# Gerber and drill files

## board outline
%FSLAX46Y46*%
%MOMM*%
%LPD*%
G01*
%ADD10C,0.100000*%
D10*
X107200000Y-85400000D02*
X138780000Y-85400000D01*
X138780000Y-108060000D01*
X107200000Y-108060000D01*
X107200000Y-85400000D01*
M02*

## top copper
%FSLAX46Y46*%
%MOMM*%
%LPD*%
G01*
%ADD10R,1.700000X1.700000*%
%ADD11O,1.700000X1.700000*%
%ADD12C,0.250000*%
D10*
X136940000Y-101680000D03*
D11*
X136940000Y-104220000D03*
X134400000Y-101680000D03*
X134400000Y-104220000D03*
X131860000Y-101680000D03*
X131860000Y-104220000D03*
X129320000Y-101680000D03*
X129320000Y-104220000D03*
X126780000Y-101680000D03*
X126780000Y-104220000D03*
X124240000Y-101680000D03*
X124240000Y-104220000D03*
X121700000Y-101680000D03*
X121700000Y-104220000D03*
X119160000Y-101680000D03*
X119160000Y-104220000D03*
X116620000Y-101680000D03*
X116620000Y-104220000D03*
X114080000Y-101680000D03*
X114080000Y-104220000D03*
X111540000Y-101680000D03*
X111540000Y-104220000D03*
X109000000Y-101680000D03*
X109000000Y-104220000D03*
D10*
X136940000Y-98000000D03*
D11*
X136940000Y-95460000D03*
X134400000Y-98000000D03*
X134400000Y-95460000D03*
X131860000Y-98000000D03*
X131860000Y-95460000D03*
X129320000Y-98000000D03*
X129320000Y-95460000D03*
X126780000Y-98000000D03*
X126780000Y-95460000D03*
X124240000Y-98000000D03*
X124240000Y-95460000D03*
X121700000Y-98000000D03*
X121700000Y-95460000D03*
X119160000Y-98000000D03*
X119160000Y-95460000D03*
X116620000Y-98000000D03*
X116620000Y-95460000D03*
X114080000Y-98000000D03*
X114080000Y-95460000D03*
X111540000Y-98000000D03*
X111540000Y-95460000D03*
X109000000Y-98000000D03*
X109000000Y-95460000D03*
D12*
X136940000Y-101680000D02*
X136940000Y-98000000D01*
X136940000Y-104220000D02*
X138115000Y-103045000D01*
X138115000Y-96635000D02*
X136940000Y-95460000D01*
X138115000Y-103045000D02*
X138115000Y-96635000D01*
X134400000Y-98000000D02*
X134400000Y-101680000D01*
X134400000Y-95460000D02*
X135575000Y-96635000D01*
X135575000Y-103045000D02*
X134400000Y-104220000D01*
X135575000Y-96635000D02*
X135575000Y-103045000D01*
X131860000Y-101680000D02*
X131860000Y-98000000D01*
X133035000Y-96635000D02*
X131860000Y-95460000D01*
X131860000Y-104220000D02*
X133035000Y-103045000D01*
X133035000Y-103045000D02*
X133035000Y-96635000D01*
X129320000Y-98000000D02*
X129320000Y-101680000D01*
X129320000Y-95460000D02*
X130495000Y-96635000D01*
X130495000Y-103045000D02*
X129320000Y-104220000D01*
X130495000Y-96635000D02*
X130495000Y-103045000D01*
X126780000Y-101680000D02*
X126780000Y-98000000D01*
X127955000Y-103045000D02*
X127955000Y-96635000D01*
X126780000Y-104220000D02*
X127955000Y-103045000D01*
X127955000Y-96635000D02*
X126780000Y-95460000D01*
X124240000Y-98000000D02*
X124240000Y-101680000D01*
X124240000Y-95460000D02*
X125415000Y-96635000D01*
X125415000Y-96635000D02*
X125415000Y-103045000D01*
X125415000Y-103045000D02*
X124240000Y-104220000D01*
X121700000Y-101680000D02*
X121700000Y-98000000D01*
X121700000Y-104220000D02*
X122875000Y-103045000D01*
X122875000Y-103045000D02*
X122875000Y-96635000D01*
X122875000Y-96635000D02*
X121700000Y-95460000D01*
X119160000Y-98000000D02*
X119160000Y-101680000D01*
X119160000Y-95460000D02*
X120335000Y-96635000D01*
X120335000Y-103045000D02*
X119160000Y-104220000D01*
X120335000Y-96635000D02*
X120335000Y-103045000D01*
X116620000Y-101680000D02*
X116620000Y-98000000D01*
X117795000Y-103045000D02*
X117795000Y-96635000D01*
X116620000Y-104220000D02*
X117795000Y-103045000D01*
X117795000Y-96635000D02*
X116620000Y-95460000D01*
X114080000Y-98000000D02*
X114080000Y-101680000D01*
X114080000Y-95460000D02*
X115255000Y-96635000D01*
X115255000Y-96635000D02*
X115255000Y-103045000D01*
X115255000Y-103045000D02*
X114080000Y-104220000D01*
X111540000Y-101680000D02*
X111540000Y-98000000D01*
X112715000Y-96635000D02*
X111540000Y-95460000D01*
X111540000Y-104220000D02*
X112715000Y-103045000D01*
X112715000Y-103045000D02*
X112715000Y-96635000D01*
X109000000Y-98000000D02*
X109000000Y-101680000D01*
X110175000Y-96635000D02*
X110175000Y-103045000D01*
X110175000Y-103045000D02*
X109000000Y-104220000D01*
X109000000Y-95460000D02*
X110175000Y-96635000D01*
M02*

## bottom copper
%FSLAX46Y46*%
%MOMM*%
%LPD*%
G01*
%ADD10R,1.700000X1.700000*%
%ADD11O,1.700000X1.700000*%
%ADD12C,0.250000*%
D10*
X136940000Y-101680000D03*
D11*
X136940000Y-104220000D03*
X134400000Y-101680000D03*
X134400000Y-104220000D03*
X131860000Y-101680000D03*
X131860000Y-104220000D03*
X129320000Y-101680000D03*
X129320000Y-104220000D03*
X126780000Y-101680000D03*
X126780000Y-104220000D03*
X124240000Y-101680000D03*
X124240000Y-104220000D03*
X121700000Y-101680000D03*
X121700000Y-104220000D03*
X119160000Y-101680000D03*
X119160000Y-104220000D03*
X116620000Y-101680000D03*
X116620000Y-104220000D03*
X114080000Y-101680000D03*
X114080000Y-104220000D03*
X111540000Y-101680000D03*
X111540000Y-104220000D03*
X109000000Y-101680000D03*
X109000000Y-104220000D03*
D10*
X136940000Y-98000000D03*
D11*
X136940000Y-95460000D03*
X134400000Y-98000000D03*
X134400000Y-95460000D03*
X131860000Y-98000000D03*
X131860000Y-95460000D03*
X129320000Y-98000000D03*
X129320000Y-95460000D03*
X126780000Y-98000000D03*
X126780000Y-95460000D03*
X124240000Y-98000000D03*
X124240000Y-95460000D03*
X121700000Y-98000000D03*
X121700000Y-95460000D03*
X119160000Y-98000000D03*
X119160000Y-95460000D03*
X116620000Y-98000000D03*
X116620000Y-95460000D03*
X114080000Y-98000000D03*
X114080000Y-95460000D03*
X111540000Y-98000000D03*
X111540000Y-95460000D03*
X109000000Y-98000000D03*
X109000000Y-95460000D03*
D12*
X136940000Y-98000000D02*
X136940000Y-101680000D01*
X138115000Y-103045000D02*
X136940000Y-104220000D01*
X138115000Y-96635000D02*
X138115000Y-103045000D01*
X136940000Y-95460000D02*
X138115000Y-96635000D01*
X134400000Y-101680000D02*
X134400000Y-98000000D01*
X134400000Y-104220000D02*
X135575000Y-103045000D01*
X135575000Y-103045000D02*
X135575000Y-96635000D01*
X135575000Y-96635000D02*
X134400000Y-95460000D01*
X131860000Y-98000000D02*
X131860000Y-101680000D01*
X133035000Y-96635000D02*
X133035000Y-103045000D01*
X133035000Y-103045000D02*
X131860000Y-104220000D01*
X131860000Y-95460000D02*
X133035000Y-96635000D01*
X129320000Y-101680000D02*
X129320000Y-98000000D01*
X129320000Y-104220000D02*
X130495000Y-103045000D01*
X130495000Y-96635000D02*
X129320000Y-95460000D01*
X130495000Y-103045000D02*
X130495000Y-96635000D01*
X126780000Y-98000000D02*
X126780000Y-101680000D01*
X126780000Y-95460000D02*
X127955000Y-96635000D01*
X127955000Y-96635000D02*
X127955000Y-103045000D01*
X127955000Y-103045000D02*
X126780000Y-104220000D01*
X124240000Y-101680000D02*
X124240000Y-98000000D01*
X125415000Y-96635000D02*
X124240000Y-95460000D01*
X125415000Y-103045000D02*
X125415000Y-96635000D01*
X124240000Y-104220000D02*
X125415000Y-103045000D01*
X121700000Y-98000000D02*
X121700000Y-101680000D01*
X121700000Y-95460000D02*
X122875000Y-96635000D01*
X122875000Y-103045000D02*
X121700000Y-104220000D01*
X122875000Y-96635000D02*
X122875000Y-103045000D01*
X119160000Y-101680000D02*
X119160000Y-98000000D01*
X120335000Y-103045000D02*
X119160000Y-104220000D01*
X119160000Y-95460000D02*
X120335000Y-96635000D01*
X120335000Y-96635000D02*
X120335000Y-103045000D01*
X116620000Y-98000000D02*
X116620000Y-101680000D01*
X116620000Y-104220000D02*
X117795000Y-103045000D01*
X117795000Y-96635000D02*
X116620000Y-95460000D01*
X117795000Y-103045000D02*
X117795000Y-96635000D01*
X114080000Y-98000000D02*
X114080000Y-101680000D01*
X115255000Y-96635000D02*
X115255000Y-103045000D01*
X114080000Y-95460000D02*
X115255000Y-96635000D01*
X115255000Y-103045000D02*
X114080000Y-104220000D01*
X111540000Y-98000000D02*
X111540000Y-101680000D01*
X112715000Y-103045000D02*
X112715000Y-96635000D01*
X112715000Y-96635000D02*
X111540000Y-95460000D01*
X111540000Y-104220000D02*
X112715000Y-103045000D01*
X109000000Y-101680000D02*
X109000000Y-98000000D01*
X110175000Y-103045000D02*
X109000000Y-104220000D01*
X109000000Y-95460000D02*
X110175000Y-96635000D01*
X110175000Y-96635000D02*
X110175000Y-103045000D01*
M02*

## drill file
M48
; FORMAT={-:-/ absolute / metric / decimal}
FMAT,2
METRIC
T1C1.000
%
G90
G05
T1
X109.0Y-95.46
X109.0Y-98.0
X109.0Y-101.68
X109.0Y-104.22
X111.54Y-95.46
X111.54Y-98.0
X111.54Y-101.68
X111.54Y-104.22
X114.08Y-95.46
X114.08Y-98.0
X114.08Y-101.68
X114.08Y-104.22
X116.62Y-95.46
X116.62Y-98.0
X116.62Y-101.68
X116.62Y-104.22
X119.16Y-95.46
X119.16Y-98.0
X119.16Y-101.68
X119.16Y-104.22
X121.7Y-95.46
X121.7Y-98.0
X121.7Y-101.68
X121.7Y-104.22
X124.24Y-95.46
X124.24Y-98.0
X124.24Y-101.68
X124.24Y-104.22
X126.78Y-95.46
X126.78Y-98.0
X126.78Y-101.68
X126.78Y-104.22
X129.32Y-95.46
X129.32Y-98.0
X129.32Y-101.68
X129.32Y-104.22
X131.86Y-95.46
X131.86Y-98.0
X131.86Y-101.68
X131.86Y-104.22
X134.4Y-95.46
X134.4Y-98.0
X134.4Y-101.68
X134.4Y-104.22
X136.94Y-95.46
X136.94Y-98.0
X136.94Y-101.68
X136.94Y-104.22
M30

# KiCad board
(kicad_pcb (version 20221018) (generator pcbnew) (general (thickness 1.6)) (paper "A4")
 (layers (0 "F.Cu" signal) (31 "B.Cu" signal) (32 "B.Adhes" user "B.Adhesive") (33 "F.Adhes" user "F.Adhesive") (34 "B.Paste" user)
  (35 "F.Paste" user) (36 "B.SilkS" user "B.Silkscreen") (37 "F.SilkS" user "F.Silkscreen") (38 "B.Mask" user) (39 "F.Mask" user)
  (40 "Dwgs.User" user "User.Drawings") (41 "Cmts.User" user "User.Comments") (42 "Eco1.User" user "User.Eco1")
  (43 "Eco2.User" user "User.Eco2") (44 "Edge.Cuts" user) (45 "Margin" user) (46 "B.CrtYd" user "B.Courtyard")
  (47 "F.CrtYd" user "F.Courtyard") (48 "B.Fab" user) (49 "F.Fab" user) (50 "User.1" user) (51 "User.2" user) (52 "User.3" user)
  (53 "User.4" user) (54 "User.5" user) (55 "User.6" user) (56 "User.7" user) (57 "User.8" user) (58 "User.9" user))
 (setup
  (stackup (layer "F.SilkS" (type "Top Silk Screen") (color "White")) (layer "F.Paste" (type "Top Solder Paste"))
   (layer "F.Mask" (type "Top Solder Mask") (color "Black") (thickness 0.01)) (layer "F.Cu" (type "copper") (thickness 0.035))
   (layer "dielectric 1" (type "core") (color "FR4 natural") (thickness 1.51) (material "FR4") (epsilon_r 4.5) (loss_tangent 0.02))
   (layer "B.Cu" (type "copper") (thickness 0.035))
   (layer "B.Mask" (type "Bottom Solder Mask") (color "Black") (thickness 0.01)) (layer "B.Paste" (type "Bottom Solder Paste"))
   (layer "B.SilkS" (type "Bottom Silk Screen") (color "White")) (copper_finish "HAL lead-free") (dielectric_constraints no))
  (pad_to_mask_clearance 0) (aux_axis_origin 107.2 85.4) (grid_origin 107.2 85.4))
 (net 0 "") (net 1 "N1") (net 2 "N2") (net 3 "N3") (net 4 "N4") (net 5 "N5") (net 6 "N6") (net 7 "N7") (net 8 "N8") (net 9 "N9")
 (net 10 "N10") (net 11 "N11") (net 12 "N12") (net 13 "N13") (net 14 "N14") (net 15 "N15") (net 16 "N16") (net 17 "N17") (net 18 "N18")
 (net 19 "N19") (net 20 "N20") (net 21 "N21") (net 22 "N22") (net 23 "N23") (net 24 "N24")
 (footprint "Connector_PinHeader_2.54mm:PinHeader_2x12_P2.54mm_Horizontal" (layer "F.Cu") (at 136.94 101.68 -90)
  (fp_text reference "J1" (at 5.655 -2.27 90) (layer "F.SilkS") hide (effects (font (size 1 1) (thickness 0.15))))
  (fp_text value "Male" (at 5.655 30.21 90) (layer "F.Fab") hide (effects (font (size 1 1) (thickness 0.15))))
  (pad "1" thru_hole rect (at 0 0 270) (size 1.7 1.7) (drill 1) (layers "*.Cu" "*.Mask") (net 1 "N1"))
  (pad "2" thru_hole oval (at 2.54 0 270) (size 1.7 1.7) (drill 1) (layers "*.Cu" "*.Mask") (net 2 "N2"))
  (pad "3" thru_hole oval (at 0 2.54 270) (size 1.7 1.7) (drill 1) (layers "*.Cu" "*.Mask") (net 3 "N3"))
  (pad "4" thru_hole oval (at 2.54 2.54 270) (size 1.7 1.7) (drill 1) (layers "*.Cu" "*.Mask") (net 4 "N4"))
  (pad "5" thru_hole oval (at 0 5.08 270) (size 1.7 1.7) (drill 1) (layers "*.Cu" "*.Mask") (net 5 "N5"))
  (pad "6" thru_hole oval (at 2.54 5.08 270) (size 1.7 1.7) (drill 1) (layers "*.Cu" "*.Mask") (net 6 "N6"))
  (pad "7" thru_hole oval (at 0 7.62 270) (size 1.7 1.7) (drill 1) (layers "*.Cu" "*.Mask") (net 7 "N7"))
  (pad "8" thru_hole oval (at 2.54 7.62 270) (size 1.7 1.7) (drill 1) (layers "*.Cu" "*.Mask") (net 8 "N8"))
  (pad "9" thru_hole oval (at 0 10.16 270) (size 1.7 1.7) (drill 1) (layers "*.Cu" "*.Mask") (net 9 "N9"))
  (pad "10" thru_hole oval (at 2.54 10.16 270) (size 1.7 1.7) (drill 1) (layers "*.Cu" "*.Mask") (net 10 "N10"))
  (pad "11" thru_hole oval (at 0 12.7 270) (size 1.7 1.7) (drill 1) (layers "*.Cu" "*.Mask") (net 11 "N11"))
  (pad "12" thru_hole oval (at 2.54 12.7 270) (size 1.7 1.7) (drill 1) (layers "*.Cu" "*.Mask") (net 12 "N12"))
  (pad "13" thru_hole oval (at 0 15.24 270) (size 1.7 1.7) (drill 1) (layers "*.Cu" "*.Mask") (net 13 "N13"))
  (pad "14" thru_hole oval (at 2.54 15.24 270) (size 1.7 1.7) (drill 1) (layers "*.Cu" "*.Mask") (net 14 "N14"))
  (pad "15" thru_hole oval (at 0 17.78 270) (size 1.7 1.7) (drill 1) (layers "*.Cu" "*.Mask") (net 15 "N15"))
  (pad "16" thru_hole oval (at 2.54 17.78 270) (size 1.7 1.7) (drill 1) (layers "*.Cu" "*.Mask") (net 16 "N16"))
  (pad "17" thru_hole oval (at 0 20.32 270) (size 1.7 1.7) (drill 1) (layers "*.Cu" "*.Mask") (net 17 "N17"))
  (pad "18" thru_hole oval (at 2.54 20.32 270) (size 1.7 1.7) (drill 1) (layers "*.Cu" "*.Mask") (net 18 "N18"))
  (pad "19" thru_hole oval (at 0 22.86 270) (size 1.7 1.7) (drill 1) (layers "*.Cu" "*.Mask") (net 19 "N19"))
  (pad "20" thru_hole oval (at 2.54 22.86 270) (size 1.7 1.7) (drill 1) (layers "*.Cu" "*.Mask") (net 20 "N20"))
  (pad "21" thru_hole oval (at 0 25.4 270) (size 1.7 1.7) (drill 1) (layers "*.Cu" "*.Mask") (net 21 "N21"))
  (pad "22" thru_hole oval (at 2.54 25.4 270) (size 1.7 1.7) (drill 1) (layers "*.Cu" "*.Mask") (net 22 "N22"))
  (pad "23" thru_hole oval (at 0 27.94 270) (size 1.7 1.7) (drill 1) (layers "*.Cu" "*.Mask") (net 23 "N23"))
  (pad "24" thru_hole oval (at 2.54 27.94 270) (size 1.7 1.7) (drill 1) (layers "*.Cu" "*.Mask") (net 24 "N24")))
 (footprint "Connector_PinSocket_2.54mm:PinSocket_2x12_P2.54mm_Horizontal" (layer "F.Cu") (at 136.94 98 -90)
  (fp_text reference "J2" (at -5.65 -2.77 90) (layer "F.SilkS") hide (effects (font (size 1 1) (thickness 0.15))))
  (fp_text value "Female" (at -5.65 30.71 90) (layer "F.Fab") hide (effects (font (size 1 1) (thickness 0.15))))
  (pad "1" thru_hole rect (at 0 0 270) (size 1.7 1.7) (drill 1) (layers "*.Cu" "*.Mask") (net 1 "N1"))
  (pad "2" thru_hole oval (at -2.54 0 270) (size 1.7 1.7) (drill 1) (layers "*.Cu" "*.Mask") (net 2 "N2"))
  (pad "3" thru_hole oval (at 0 2.54 270) (size 1.7 1.7) (drill 1) (layers "*.Cu" "*.Mask") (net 3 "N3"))
  (pad "4" thru_hole oval (at -2.54 2.54 270) (size 1.7 1.7) (drill 1) (layers "*.Cu" "*.Mask") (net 4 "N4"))
  (pad "5" thru_hole oval (at 0 5.08 270) (size 1.7 1.7) (drill 1) (layers "*.Cu" "*.Mask") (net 5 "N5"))
  (pad "6" thru_hole oval (at -2.54 5.08 270) (size 1.7 1.7) (drill 1) (layers "*.Cu" "*.Mask") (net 6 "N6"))
  (pad "7" thru_hole oval (at 0 7.62 270) (size 1.7 1.7) (drill 1) (layers "*.Cu" "*.Mask") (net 7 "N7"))
  (pad "8" thru_hole oval (at -2.54 7.62 270) (size 1.7 1.7) (drill 1) (layers "*.Cu" "*.Mask") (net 8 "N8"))
  (pad "9" thru_hole oval (at 0 10.16 270) (size 1.7 1.7) (drill 1) (layers "*.Cu" "*.Mask") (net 9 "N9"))
  (pad "10" thru_hole oval (at -2.54 10.16 270) (size 1.7 1.7) (drill 1) (layers "*.Cu" "*.Mask") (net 10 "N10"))
  (pad "11" thru_hole oval (at 0 12.7 270) (size 1.7 1.7) (drill 1) (layers "*.Cu" "*.Mask") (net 11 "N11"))
  (pad "12" thru_hole oval (at -2.54 12.7 270) (size 1.7 1.7) (drill 1) (layers "*.Cu" "*.Mask") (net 12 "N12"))
  (pad "13" thru_hole oval (at 0 15.24 270) (size 1.7 1.7) (drill 1) (layers "*.Cu" "*.Mask") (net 13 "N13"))
  (pad "14" thru_hole oval (at -2.54 15.24 270) (size 1.7 1.7) (drill 1) (layers "*.Cu" "*.Mask") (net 14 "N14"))
  (pad "15" thru_hole oval (at 0 17.78 270) (size 1.7 1.7) (drill 1) (layers "*.Cu" "*.Mask") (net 15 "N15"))
  (pad "16" thru_hole oval (at -2.54 17.78 270) (size 1.7 1.7) (drill 1) (layers "*.Cu" "*.Mask") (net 16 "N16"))
  (pad "17" thru_hole oval (at 0 20.32 270) (size 1.7 1.7) (drill 1) (layers "*.Cu" "*.Mask") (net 17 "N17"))
  (pad "18" thru_hole oval (at -2.54 20.32 270) (size 1.7 1.7) (drill 1) (layers "*.Cu" "*.Mask") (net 18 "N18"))
  (pad "19" thru_hole oval (at 0 22.86 270) (size 1.7 1.7) (drill 1) (layers "*.Cu" "*.Mask") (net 19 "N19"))
  (pad "20" thru_hole oval (at -2.54 22.86 270) (size 1.7 1.7) (drill 1) (layers "*.Cu" "*.Mask") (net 20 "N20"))
  (pad "21" thru_hole oval (at 0 25.4 270) (size 1.7 1.7) (drill 1) (layers "*.Cu" "*.Mask") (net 21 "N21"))
  (pad "22" thru_hole oval (at -2.54 25.4 270) (size 1.7 1.7) (drill 1) (layers "*.Cu" "*.Mask") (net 22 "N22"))
  (pad "23" thru_hole oval (at 0 27.94 270) (size 1.7 1.7) (drill 1) (layers "*.Cu" "*.Mask") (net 23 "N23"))
  (pad "24" thru_hole oval (at -2.54 27.94 270) (size 1.7 1.7) (drill 1) (layers "*.Cu" "*.Mask") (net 24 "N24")))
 (gr_rect (start 107.2 85.4) (end 138.78 108.06) (stroke (width 0.1) (type default)) (fill none) (layer "Edge.Cuts"))
 (segment (start 136.94 101.68) (end 136.94 98) (width 0.25) (layer "F.Cu") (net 1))
 (segment (start 136.94 98) (end 136.94 101.68) (width 0.25) (layer "B.Cu") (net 1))
 (segment (start 136.94 104.22) (end 138.115 103.045) (width 0.25) (layer "F.Cu") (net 2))
 (segment (start 138.115 96.635) (end 136.94 95.46) (width 0.25) (layer "F.Cu") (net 2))
 (segment (start 138.115 103.045) (end 138.115 96.635) (width 0.25) (layer "F.Cu") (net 2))
 (segment (start 138.115 103.045) (end 136.94 104.22) (width 0.25) (layer "B.Cu") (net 2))
 (segment (start 138.115 96.635) (end 138.115 103.045) (width 0.25) (layer "B.Cu") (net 2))
 (segment (start 136.94 95.46) (end 138.115 96.635) (width 0.25) (layer "B.Cu") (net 2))
 (segment (start 134.4 98) (end 134.4 101.68) (width 0.25) (layer "F.Cu") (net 3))
 (segment (start 134.4 101.68) (end 134.4 98) (width 0.25) (layer "B.Cu") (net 3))
 (segment (start 134.4 95.46) (end 135.575 96.635) (width 0.25) (layer "F.Cu") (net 4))
 (segment (start 135.575 103.045) (end 134.4 104.22) (width 0.25) (layer "F.Cu") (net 4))
 (segment (start 135.575 96.635) (end 135.575 103.045) (width 0.25) (layer "F.Cu") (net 4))
 (segment (start 134.4 104.22) (end 135.575 103.045) (width 0.25) (layer "B.Cu") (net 4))
 (segment (start 135.575 103.045) (end 135.575 96.635) (width 0.25) (layer "B.Cu") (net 4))
 (segment (start 135.575 96.635) (end 134.4 95.46) (width 0.25) (layer "B.Cu") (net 4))
 (segment (start 131.86 101.68) (end 131.86 98) (width 0.25) (layer "F.Cu") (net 5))
 (segment (start 131.86 98) (end 131.86 101.68) (width 0.25) (layer "B.Cu") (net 5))
 (segment (start 133.035 96.635) (end 131.86 95.46) (width 0.25) (layer "F.Cu") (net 6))
 (segment (start 131.86 104.22) (end 133.035 103.045) (width 0.25) (layer "F.Cu") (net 6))
 (segment (start 133.035 103.045) (end 133.035 96.635) (width 0.25) (layer "F.Cu") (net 6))
 (segment (start 133.035 96.635) (end 133.035 103.045) (width 0.25) (layer "B.Cu") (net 6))
 (segment (start 133.035 103.045) (end 131.86 104.22) (width 0.25) (layer "B.Cu") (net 6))
 (segment (start 131.86 95.46) (end 133.035 96.635) (width 0.25) (layer "B.Cu") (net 6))
 (segment (start 129.32 98) (end 129.32 101.68) (width 0.25) (layer "F.Cu") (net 7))
 (segment (start 129.32 101.68) (end 129.32 98) (width 0.25) (layer "B.Cu") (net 7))
 (segment (start 129.32 95.46) (end 130.495 96.635) (width 0.25) (layer "F.Cu") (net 8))
 (segment (start 130.495 103.045) (end 129.32 104.22) (width 0.25) (layer "F.Cu") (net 8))
 (segment (start 130.495 96.635) (end 130.495 103.045) (width 0.25) (layer "F.Cu") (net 8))
 (segment (start 129.32 104.22) (end 130.495 103.045) (width 0.25) (layer "B.Cu") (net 8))
 (segment (start 130.495 96.635) (end 129.32 95.46) (width 0.25) (layer "B.Cu") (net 8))
 (segment (start 130.495 103.045) (end 130.495 96.635) (width 0.25) (layer "B.Cu") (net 8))
 (segment (start 126.78 101.68) (end 126.78 98) (width 0.25) (layer "F.Cu") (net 9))
 (segment (start 126.78 98) (end 126.78 101.68) (width 0.25) (layer "B.Cu") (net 9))
 (segment (start 127.955 103.045) (end 127.955 96.635) (width 0.25) (layer "F.Cu") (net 10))
 (segment (start 126.78 104.22) (end 127.955 103.045) (width 0.25) (layer "F.Cu") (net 10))
 (segment (start 127.955 96.635) (end 126.78 95.46) (width 0.25) (layer "F.Cu") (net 10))
 (segment (start 126.78 95.46) (end 127.955 96.635) (width 0.25) (layer "B.Cu") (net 10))
 (segment (start 127.955 96.635) (end 127.955 103.045) (width 0.25) (layer "B.Cu") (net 10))
 (segment (start 127.955 103.045) (end 126.78 104.22) (width 0.25) (layer "B.Cu") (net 10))
 (segment (start 124.24 98) (end 124.24 101.68) (width 0.25) (layer "F.Cu") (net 11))
 (segment (start 124.24 101.68) (end 124.24 98) (width 0.25) (layer "B.Cu") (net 11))
 (segment (start 124.24 95.46) (end 125.415 96.635) (width 0.25) (layer "F.Cu") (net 12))
 (segment (start 125.415 96.635) (end 125.415 103.045) (width 0.25) (layer "F.Cu") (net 12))
 (segment (start 125.415 103.045) (end 124.24 104.22) (width 0.25) (layer "F.Cu") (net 12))
 (segment (start 125.415 96.635) (end 124.24 95.46) (width 0.25) (layer "B.Cu") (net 12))
 (segment (start 125.415 103.045) (end 125.415 96.635) (width 0.25) (layer "B.Cu") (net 12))
 (segment (start 124.24 104.22) (end 125.415 103.045) (width 0.25) (layer "B.Cu") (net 12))
 (segment (start 121.7 101.68) (end 121.7 98) (width 0.25) (layer "F.Cu") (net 13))
 (segment (start 121.7 98) (end 121.7 101.68) (width 0.25) (layer "B.Cu") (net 13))
 (segment (start 121.7 104.22) (end 122.875 103.045) (width 0.25) (layer "F.Cu") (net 14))
 (segment (start 122.875 103.045) (end 122.875 96.635) (width 0.25) (layer "F.Cu") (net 14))
 (segment (start 122.875 96.635) (end 121.7 95.46) (width 0.25) (layer "F.Cu") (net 14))
 (segment (start 121.7 95.46) (end 122.875 96.635) (width 0.25) (layer "B.Cu") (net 14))
 (segment (start 122.875 103.045) (end 121.7 104.22) (width 0.25) (layer "B.Cu") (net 14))
 (segment (start 122.875 96.635) (end 122.875 103.045) (width 0.25) (layer "B.Cu") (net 14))
 (segment (start 119.16 98) (end 119.16 101.68) (width 0.25) (layer "F.Cu") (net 15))
 (segment (start 119.16 101.68) (end 119.16 98) (width 0.25) (layer "B.Cu") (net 15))
 (segment (start 119.16 95.46) (end 120.335 96.635) (width 0.25) (layer "F.Cu") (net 16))
 (segment (start 120.335 103.045) (end 119.16 104.22) (width 0.25) (layer "F.Cu") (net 16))
 (segment (start 120.335 96.635) (end 120.335 103.045) (width 0.25) (layer "F.Cu") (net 16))
 (segment (start 120.335 103.045) (end 119.16 104.22) (width 0.25) (layer "B.Cu") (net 16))
 (segment (start 119.16 95.46) (end 120.335 96.635) (width 0.25) (layer "B.Cu") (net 16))
 (segment (start 120.335 96.635) (end 120.335 103.045) (width 0.25) (layer "B.Cu") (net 16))
 (segment (start 116.62 101.68) (end 116.62 98) (width 0.25) (layer "F.Cu") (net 17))
 (segment (start 116.62 98) (end 116.62 101.68) (width 0.25) (layer "B.Cu") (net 17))
 (segment (start 117.795 103.045) (end 117.795 96.635) (width 0.25) (layer "F.Cu") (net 18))
 (segment (start 116.62 104.22) (end 117.795 103.045) (width 0.25) (layer "F.Cu") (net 18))
 (segment (start 117.795 96.635) (end 116.62 95.46) (width 0.25) (layer "F.Cu") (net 18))
 (segment (start 116.62 104.22) (end 117.795 103.045) (width 0.25) (layer "B.Cu") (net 18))
 (segment (start 117.795 96.635) (end 116.62 95.46) (width 0.25) (layer "B.Cu") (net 18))
 (segment (start 117.795 103.045) (end 117.795 96.635) (width 0.25) (layer "B.Cu") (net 18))
 (segment (start 114.08 98) (end 114.08 101.68) (width 0.25) (layer "F.Cu") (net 19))
 (segment (start 114.08 98) (end 114.08 101.68) (width 0.25) (layer "B.Cu") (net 19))
 (segment (start 114.08 95.46) (end 115.255 96.635) (width 0.25) (layer "F.Cu") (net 20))
 (segment (start 115.255 96.635) (end 115.255 103.045) (width 0.25) (layer "F.Cu") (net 20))
 (segment (start 115.255 103.045) (end 114.08 104.22) (width 0.25) (layer "F.Cu") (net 20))
 (segment (start 115.255 96.635) (end 115.255 103.045) (width 0.25) (layer "B.Cu") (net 20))
 (segment (start 114.08 95.46) (end 115.255 96.635) (width 0.25) (layer "B.Cu") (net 20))
 (segment (start 115.255 103.045) (end 114.08 104.22) (width 0.25) (layer "B.Cu") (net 20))
 (segment (start 111.54 101.68) (end 111.54 98) (width 0.25) (layer "F.Cu") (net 21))
 (segment (start 111.54 98) (end 111.54 101.68) (width 0.25) (layer "B.Cu") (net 21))
 (segment (start 112.715 96.635) (end 111.54 95.46) (width 0.25) (layer "F.Cu") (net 22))
 (segment (start 111.54 104.22) (end 112.715 103.045) (width 0.25) (layer "F.Cu") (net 22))
 (segment (start 112.715 103.045) (end 112.715 96.635) (width 0.25) (layer "F.Cu") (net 22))
 (segment (start 112.715 103.045) (end 112.715 96.635) (width 0.25) (layer "B.Cu") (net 22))
 (segment (start 112.715 96.635) (end 111.54 95.46) (width 0.25) (layer "B.Cu") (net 22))
 (segment (start 111.54 104.22) (end 112.715 103.045) (width 0.25) (layer "B.Cu") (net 22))
 (segment (start 109 98) (end 109 101.68) (width 0.25) (layer "F.Cu") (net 23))
 (segment (start 109 101.68) (end 109 98) (width 0.25) (layer "B.Cu") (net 23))
 (segment (start 110.175 96.635) (end 110.175 103.045) (width 0.25) (layer "F.Cu") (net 24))
 (segment (start 110.175 103.045) (end 109 104.22) (width 0.25) (layer "F.Cu") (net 24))
 (segment (start 109 95.46) (end 110.175 96.635) (width 0.25) (layer "F.Cu") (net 24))
 (segment (start 110.175 103.045) (end 109 104.22) (width 0.25) (layer "B.Cu") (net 24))
 (segment (start 109 95.46) (end 110.175 96.635) (width 0.25) (layer "B.Cu") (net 24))
 (segment (start 110.175 96.635) (end 110.175 103.045) (width 0.25) (layer "B.Cu") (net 24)))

